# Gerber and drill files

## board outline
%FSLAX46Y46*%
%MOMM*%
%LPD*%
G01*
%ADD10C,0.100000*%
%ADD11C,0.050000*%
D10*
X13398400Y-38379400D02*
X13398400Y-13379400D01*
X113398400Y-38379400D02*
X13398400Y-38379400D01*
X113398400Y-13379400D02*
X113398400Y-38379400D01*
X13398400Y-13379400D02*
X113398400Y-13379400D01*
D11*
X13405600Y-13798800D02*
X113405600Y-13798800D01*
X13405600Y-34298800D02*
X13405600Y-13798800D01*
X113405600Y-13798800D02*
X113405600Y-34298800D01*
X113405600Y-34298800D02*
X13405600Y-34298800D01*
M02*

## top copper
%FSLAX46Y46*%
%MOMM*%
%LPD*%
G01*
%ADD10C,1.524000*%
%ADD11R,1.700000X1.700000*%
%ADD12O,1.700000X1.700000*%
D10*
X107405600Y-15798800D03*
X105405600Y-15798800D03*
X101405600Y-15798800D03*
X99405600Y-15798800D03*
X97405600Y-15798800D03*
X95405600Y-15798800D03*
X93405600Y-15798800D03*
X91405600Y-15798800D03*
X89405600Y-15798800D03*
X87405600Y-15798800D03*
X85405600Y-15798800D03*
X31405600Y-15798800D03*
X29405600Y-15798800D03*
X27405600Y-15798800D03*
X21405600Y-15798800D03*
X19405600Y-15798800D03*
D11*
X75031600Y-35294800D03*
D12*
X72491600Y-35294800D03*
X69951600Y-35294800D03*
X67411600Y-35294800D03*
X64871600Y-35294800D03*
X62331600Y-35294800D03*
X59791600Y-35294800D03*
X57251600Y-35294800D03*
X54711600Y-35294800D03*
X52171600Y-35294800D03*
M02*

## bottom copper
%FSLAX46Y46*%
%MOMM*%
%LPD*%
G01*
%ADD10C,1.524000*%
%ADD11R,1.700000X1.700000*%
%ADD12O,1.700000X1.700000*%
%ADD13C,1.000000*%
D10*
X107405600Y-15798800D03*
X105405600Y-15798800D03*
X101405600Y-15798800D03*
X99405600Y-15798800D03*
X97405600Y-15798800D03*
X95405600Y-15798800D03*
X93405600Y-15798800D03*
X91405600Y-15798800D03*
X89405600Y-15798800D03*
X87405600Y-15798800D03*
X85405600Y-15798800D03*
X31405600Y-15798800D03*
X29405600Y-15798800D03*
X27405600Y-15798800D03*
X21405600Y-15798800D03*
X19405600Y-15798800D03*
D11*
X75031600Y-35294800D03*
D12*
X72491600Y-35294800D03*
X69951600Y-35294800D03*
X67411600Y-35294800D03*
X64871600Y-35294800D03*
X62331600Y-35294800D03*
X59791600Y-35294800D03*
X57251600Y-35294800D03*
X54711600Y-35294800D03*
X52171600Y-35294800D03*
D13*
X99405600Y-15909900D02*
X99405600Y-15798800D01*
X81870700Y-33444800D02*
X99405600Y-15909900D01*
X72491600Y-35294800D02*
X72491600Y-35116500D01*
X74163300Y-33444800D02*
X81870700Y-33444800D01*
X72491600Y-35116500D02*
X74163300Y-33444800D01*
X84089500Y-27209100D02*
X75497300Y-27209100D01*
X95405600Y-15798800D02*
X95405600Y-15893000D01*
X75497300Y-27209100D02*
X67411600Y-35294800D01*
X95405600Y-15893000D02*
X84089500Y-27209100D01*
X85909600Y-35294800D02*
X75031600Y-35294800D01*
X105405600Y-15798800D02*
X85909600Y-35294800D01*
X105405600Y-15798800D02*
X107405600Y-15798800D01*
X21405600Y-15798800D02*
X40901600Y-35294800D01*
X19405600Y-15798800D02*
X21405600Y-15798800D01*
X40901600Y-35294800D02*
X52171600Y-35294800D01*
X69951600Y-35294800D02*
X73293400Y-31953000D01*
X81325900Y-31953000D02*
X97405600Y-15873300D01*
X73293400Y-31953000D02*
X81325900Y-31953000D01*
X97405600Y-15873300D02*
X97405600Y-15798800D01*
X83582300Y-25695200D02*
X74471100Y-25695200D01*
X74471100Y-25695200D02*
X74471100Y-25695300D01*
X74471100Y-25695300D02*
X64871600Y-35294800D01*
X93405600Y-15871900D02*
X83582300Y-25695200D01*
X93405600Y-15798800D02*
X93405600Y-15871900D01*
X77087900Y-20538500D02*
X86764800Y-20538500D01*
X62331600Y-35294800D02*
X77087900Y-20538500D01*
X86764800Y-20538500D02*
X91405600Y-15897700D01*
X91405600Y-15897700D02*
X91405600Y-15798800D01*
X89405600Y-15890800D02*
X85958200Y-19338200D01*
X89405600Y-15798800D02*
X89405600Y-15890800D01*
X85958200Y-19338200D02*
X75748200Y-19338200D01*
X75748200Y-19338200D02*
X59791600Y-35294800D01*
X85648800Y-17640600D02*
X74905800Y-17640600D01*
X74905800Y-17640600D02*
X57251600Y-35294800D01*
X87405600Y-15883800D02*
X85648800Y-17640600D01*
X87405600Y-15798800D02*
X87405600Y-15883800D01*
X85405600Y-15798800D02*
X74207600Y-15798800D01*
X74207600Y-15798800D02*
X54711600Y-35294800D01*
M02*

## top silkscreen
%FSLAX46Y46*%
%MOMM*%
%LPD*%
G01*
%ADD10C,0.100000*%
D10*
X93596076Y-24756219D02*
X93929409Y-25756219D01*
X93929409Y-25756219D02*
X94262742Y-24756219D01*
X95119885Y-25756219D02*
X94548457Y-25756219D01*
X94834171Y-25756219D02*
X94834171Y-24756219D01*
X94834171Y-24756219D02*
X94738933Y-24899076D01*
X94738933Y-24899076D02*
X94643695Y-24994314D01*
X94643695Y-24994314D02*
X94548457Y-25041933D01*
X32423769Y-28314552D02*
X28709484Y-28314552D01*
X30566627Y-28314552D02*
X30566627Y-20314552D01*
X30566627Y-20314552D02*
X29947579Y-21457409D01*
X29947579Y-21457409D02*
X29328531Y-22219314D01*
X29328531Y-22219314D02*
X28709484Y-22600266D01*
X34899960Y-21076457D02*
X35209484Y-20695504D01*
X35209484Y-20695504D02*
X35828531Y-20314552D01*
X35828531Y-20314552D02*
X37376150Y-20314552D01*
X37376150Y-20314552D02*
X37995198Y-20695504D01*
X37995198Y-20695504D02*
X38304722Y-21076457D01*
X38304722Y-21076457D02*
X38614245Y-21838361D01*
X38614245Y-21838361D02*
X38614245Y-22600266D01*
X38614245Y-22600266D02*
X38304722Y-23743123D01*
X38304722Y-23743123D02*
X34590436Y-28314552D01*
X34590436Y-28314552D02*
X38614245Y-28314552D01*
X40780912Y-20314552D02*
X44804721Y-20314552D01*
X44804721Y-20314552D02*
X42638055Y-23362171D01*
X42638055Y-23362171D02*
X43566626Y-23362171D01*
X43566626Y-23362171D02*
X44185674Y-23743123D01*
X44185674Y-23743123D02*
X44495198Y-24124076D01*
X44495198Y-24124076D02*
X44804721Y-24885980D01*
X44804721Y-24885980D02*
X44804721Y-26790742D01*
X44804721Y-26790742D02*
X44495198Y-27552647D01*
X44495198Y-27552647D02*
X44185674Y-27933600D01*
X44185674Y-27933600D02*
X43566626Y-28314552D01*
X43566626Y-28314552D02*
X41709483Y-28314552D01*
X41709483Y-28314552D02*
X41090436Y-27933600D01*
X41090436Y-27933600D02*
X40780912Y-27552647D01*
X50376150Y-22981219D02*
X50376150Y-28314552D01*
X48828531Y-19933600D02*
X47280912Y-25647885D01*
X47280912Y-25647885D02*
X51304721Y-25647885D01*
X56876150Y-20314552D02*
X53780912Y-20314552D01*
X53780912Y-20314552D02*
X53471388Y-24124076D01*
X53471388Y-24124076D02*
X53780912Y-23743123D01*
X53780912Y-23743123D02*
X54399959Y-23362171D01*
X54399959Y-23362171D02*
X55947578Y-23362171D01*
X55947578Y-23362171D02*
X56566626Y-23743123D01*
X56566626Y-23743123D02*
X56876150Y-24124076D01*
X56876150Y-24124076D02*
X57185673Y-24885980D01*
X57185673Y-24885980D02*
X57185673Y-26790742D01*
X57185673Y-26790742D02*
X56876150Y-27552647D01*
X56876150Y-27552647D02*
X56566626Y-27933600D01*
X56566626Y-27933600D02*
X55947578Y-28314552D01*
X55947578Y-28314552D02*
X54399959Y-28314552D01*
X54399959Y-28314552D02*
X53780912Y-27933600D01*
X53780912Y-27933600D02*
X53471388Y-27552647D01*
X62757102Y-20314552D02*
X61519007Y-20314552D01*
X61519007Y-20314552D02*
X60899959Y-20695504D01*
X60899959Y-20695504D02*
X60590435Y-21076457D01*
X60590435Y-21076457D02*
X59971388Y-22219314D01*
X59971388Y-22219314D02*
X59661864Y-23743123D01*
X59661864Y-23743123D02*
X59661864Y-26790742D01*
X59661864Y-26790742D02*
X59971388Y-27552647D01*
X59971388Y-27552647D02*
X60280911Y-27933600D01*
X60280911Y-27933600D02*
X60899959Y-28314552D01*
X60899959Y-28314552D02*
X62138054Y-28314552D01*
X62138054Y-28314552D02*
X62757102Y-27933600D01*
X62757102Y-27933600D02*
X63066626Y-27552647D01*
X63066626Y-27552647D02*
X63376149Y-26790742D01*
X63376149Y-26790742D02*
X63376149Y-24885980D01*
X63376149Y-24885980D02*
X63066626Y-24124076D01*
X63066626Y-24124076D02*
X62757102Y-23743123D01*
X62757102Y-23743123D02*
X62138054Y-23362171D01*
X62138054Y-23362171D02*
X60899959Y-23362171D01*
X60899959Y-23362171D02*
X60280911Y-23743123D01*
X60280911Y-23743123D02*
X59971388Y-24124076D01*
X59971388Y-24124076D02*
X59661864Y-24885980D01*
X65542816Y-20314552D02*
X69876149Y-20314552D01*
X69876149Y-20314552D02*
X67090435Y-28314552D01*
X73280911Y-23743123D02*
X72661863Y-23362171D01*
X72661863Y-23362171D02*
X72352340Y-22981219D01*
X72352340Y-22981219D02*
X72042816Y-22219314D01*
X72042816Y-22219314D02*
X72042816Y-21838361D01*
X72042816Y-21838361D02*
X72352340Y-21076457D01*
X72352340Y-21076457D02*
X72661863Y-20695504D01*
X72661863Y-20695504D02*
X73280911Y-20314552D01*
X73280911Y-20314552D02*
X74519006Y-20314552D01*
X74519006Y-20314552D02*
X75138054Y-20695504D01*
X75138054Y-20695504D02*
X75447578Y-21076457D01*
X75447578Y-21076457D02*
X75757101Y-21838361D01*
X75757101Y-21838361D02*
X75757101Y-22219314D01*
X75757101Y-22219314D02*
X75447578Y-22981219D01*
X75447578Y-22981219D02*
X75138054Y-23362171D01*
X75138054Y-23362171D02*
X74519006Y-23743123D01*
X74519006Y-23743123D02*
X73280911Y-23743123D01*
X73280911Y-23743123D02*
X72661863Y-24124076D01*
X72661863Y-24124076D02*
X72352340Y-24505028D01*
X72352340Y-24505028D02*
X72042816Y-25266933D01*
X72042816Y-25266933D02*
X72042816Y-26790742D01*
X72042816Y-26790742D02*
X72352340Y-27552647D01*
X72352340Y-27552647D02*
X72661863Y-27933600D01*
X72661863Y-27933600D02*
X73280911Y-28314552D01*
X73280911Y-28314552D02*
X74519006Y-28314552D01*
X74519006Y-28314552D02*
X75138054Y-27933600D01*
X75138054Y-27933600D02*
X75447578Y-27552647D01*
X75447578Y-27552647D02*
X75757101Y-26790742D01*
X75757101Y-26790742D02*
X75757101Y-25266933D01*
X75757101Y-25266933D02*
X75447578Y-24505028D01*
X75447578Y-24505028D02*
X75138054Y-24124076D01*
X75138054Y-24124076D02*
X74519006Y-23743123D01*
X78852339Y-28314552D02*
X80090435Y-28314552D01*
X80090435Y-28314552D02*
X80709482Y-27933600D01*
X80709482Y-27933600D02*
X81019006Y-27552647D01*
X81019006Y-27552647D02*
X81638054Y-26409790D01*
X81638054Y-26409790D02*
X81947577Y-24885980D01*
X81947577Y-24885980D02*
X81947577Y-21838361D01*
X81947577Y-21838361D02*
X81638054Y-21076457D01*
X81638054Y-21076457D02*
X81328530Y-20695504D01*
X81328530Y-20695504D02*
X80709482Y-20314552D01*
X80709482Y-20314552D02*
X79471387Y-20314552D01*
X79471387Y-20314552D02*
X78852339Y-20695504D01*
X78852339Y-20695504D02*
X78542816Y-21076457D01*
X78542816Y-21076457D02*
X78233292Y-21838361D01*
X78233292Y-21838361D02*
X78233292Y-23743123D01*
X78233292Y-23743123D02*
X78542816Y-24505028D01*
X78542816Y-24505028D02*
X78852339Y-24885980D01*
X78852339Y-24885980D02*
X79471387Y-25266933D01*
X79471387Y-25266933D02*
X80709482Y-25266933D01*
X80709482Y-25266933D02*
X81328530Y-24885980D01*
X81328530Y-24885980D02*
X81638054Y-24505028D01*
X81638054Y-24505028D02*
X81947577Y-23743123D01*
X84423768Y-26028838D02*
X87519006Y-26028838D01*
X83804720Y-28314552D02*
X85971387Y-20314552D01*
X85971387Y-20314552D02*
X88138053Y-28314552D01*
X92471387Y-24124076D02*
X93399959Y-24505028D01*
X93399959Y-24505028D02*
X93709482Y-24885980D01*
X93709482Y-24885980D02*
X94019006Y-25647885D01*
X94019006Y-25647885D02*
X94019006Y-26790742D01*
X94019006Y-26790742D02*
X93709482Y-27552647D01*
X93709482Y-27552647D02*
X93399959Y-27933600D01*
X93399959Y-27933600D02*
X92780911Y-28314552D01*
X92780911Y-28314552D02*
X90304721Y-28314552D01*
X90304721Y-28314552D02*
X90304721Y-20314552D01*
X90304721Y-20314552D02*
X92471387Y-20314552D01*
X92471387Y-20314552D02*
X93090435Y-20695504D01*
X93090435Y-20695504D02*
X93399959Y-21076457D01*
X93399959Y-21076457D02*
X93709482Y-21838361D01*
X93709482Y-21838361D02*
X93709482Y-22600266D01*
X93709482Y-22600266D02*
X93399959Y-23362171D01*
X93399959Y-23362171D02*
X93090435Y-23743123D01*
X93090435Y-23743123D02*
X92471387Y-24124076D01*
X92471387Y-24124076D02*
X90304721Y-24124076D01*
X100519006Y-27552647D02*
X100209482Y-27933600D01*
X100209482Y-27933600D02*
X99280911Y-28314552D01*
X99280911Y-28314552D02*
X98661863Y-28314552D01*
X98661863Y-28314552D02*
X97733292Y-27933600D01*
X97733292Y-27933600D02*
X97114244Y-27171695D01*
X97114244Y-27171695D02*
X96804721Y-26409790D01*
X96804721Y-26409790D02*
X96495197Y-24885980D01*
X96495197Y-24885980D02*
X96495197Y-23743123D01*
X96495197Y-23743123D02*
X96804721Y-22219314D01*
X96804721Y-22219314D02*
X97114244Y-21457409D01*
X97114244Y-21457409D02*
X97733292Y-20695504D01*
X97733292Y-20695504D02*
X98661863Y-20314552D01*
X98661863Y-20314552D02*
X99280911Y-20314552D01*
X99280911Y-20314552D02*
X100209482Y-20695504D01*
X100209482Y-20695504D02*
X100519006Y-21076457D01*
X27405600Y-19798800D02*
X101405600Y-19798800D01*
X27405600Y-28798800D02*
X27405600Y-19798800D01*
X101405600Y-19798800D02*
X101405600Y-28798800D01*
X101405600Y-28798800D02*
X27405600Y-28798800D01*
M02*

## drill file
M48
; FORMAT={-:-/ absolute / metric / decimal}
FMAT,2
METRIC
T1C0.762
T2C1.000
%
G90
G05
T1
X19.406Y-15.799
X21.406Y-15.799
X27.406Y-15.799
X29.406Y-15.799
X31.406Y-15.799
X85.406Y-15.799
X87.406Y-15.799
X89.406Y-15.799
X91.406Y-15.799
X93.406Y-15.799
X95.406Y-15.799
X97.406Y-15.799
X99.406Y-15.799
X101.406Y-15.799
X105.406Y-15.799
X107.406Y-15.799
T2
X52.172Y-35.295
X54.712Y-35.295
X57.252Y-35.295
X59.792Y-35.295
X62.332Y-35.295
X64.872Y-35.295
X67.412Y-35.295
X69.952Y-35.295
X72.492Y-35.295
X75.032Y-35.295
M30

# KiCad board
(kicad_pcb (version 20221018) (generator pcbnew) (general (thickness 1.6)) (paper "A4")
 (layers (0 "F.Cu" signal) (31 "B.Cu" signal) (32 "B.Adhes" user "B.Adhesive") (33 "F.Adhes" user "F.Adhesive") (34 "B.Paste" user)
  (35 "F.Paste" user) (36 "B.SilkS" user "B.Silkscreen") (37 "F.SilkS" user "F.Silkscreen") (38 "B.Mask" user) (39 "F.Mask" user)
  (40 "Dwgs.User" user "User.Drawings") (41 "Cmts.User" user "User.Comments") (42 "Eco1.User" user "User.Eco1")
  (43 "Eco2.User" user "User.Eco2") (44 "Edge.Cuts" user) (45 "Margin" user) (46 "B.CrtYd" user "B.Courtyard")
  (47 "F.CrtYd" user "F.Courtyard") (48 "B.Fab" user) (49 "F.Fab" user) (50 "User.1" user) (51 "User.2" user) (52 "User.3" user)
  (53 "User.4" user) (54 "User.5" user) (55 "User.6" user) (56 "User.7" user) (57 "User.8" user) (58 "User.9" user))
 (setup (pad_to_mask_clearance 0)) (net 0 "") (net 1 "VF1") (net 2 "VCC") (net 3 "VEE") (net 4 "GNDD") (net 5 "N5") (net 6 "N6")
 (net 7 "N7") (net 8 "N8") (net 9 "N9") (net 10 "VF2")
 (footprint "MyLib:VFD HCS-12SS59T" (layer "F.Cu") (at 13.3056 13.9988)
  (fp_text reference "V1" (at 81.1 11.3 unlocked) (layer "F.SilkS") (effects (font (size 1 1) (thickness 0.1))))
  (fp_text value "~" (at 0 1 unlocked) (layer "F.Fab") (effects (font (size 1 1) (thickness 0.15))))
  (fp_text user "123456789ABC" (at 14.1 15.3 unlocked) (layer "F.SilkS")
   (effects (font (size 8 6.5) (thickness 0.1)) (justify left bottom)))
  (fp_line (start 14.1 5.8) (end 88.1 5.8) (stroke (width 0.1) (type default)) (layer "F.SilkS"))
  (fp_line (start 14.1 14.8) (end 14.1 5.8) (stroke (width 0.1) (type default)) (layer "F.SilkS"))
  (fp_line (start 88.1 5.8) (end 88.1 14.8) (stroke (width 0.1) (type default)) (layer "F.SilkS"))
  (fp_line (start 88.1 14.8) (end 14.1 14.8) (stroke (width 0.1) (type default)) (layer "F.SilkS"))
  (fp_line (start 0.1 -0.2) (end 100.1 -0.2) (stroke (width 0.05) (type default)) (layer "Edge.Cuts"))
  (fp_line (start 0.1 20.3) (end 0.1 -0.2) (stroke (width 0.05) (type default)) (layer "Edge.Cuts"))
  (fp_line (start 100.1 -0.2) (end 100.1 20.3) (stroke (width 0.05) (type default)) (layer "Edge.Cuts"))
  (fp_line (start 100.1 20.3) (end 0.1 20.3) (stroke (width 0.05) (type default)) (layer "Edge.Cuts"))
  (pad "1" thru_hole circle (at 94.1 1.8) (size 1.524 1.524) (drill 0.762) (layers "*.Cu" "*.Mask") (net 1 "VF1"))
  (pad "2" thru_hole circle (at 92.1 1.8) (size 1.524 1.524) (drill 0.762) (layers "*.Cu" "*.Mask") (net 1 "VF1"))
  (pad "4" thru_hole circle (at 88.1 1.8) (size 1.524 1.524) (drill 0.762) (layers "*.Cu" "*.Mask"))
  (pad "5" thru_hole circle (at 86.1 1.8) (size 1.524 1.524) (drill 0.762) (layers "*.Cu" "*.Mask") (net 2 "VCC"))
  (pad "6" thru_hole circle (at 84.1 1.8) (size 1.524 1.524) (drill 0.762) (layers "*.Cu" "*.Mask") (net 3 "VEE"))
  (pad "7" thru_hole circle (at 82.1 1.8) (size 1.524 1.524) (drill 0.762) (layers "*.Cu" "*.Mask") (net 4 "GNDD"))
  (pad "8" thru_hole circle (at 80.1 1.8) (size 1.524 1.524) (drill 0.762) (layers "*.Cu" "*.Mask") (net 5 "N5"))
  (pad "9" thru_hole circle (at 78.1 1.8) (size 1.524 1.524) (drill 0.762) (layers "*.Cu" "*.Mask") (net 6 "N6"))
  (pad "10" thru_hole circle (at 76.1 1.8) (size 1.524 1.524) (drill 0.762) (layers "*.Cu" "*.Mask") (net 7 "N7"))
  (pad "11" thru_hole circle (at 74.1 1.8) (size 1.524 1.524) (drill 0.762) (layers "*.Cu" "*.Mask") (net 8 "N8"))
  (pad "12" thru_hole circle (at 72.1 1.8) (size 1.524 1.524) (drill 0.762) (layers "*.Cu" "*.Mask") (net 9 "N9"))
  (pad "39" thru_hole circle (at 18.1 1.8) (size 1.524 1.524) (drill 0.762) (layers "*.Cu" "*.Mask"))
  (pad "40" thru_hole circle (at 16.1 1.8) (size 1.524 1.524) (drill 0.762) (layers "*.Cu" "*.Mask"))
  (pad "41" thru_hole circle (at 14.1 1.8) (size 1.524 1.524) (drill 0.762) (layers "*.Cu" "*.Mask"))
  (pad "44" thru_hole circle (at 8.1 1.8) (size 1.524 1.524) (drill 0.762) (layers "*.Cu" "*.Mask") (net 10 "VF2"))
  (pad "45" thru_hole circle (at 6.1 1.8) (size 1.524 1.524) (drill 0.762) (layers "*.Cu" "*.Mask") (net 10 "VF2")))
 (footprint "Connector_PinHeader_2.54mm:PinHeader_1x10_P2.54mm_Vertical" (layer "B.Cu") (at 75.0316 35.2948 90)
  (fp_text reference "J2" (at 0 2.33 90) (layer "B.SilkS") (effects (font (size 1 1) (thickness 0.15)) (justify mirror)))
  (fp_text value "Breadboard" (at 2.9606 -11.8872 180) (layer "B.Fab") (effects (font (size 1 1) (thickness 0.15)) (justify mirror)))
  (pad "1" thru_hole rect (at 0 0 90) (size 1.7 1.7) (drill 1) (layers "*.Cu" "*.Mask") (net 1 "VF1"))
  (pad "2" thru_hole oval (at 0 -2.54 90) (size 1.7 1.7) (drill 1) (layers "*.Cu" "*.Mask") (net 2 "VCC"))
  (pad "3" thru_hole oval (at 0 -5.08 90) (size 1.7 1.7) (drill 1) (layers "*.Cu" "*.Mask") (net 3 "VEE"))
  (pad "4" thru_hole oval (at 0 -7.62 90) (size 1.7 1.7) (drill 1) (layers "*.Cu" "*.Mask") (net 4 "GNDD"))
  (pad "5" thru_hole oval (at 0 -10.16 90) (size 1.7 1.7) (drill 1) (layers "*.Cu" "*.Mask") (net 5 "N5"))
  (pad "6" thru_hole oval (at 0 -12.7 90) (size 1.7 1.7) (drill 1) (layers "*.Cu" "*.Mask") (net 6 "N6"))
  (pad "7" thru_hole oval (at 0 -15.24 90) (size 1.7 1.7) (drill 1) (layers "*.Cu" "*.Mask") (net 7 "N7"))
  (pad "8" thru_hole oval (at 0 -17.78 90) (size 1.7 1.7) (drill 1) (layers "*.Cu" "*.Mask") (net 8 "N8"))
  (pad "9" thru_hole oval (at 0 -20.32 90) (size 1.7 1.7) (drill 1) (layers "*.Cu" "*.Mask") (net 9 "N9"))
  (pad "10" thru_hole oval (at 0 -22.86 90) (size 1.7 1.7) (drill 1) (layers "*.Cu" "*.Mask") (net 10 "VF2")))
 (gr_line (start 13.3984 38.3794) (end 13.3984 13.3794) (stroke (width 0.1) (type default)) (layer "Edge.Cuts"))
 (gr_line (start 113.3984 38.3794) (end 13.3984 38.3794) (stroke (width 0.1) (type default)) (layer "Edge.Cuts"))
 (gr_line (start 113.3984 13.3794) (end 113.3984 38.3794) (stroke (width 0.1) (type default)) (layer "Edge.Cuts"))
 (gr_line (start 13.3984 13.3794) (end 113.3984 13.3794) (stroke (width 0.1) (type default)) (layer "Edge.Cuts"))
 (segment (start 99.4056 15.9099) (end 99.4056 15.7988) (width 1) (layer "B.Cu") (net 2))
 (segment (start 81.8707 33.4448) (end 99.4056 15.9099) (width 1) (layer "B.Cu") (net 2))
 (segment (start 72.4916 35.2948) (end 72.4916 35.1165) (width 1) (layer "B.Cu") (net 2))
 (segment (start 74.1633 33.4448) (end 81.8707 33.4448) (width 1) (layer "B.Cu") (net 2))
 (segment (start 72.4916 35.1165) (end 74.1633 33.4448) (width 1) (layer "B.Cu") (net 2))
 (segment (start 84.0895 27.2091) (end 75.4973 27.2091) (width 1) (layer "B.Cu") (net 4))
 (segment (start 95.4056 15.7988) (end 95.4056 15.893) (width 1) (layer "B.Cu") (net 4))
 (segment (start 75.4973 27.2091) (end 67.4116 35.2948) (width 1) (layer "B.Cu") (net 4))
 (segment (start 95.4056 15.893) (end 84.0895 27.2091) (width 1) (layer "B.Cu") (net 4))
 (segment (start 85.9096 35.2948) (end 75.0316 35.2948) (width 1) (layer "B.Cu") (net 1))
 (segment (start 105.4056 15.7988) (end 85.9096 35.2948) (width 1) (layer "B.Cu") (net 1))
 (segment (start 105.4056 15.7988) (end 107.4056 15.7988) (width 1) (layer "B.Cu") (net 1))
 (segment (start 21.4056 15.7988) (end 40.9016 35.2948) (width 1) (layer "B.Cu") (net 10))
 (segment (start 19.4056 15.7988) (end 21.4056 15.7988) (width 1) (layer "B.Cu") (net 10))
 (segment (start 40.9016 35.2948) (end 52.1716 35.2948) (width 1) (layer "B.Cu") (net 10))
 (segment (start 69.9516 35.2948) (end 73.2934 31.953) (width 1) (layer "B.Cu") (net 3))
 (segment (start 81.3259 31.953) (end 97.4056 15.8733) (width 1) (layer "B.Cu") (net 3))
 (segment (start 73.2934 31.953) (end 81.3259 31.953) (width 1) (layer "B.Cu") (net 3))
 (segment (start 97.4056 15.8733) (end 97.4056 15.7988) (width 1) (layer "B.Cu") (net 3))
 (segment (start 83.5823 25.6952) (end 74.4711 25.6952) (width 1) (layer "B.Cu") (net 5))
 (segment (start 74.4711 25.6952) (end 74.4711 25.6953) (width 1) (layer "B.Cu") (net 5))
 (segment (start 74.4711 25.6953) (end 64.8716 35.2948) (width 1) (layer "B.Cu") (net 5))
 (segment (start 93.4056 15.8719) (end 83.5823 25.6952) (width 1) (layer "B.Cu") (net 5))
 (segment (start 93.4056 15.7988) (end 93.4056 15.8719) (width 1) (layer "B.Cu") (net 5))
 (segment (start 77.0879 20.5385) (end 86.7648 20.5385) (width 1) (layer "B.Cu") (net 6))
 (segment (start 62.3316 35.2948) (end 77.0879 20.5385) (width 1) (layer "B.Cu") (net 6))
 (segment (start 86.7648 20.5385) (end 91.4056 15.8977) (width 1) (layer "B.Cu") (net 6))
 (segment (start 91.4056 15.8977) (end 91.4056 15.7988) (width 1) (layer "B.Cu") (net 6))
 (segment (start 89.4056 15.8908) (end 85.9582 19.3382) (width 1) (layer "B.Cu") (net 7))
 (segment (start 89.4056 15.7988) (end 89.4056 15.8908) (width 1) (layer "B.Cu") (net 7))
 (segment (start 85.9582 19.3382) (end 75.7482 19.3382) (width 1) (layer "B.Cu") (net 7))
 (segment (start 75.7482 19.3382) (end 59.7916 35.2948) (width 1) (layer "B.Cu") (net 7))
 (segment (start 85.6488 17.6406) (end 74.9058 17.6406) (width 1) (layer "B.Cu") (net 8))
 (segment (start 74.9058 17.6406) (end 57.2516 35.2948) (width 1) (layer "B.Cu") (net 8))
 (segment (start 87.4056 15.8838) (end 85.6488 17.6406) (width 1) (layer "B.Cu") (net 8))
 (segment (start 87.4056 15.7988) (end 87.4056 15.8838) (width 1) (layer "B.Cu") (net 8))
 (segment (start 85.4056 15.7988) (end 74.2076 15.7988) (width 1) (layer "B.Cu") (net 9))
 (segment (start 74.2076 15.7988) (end 54.7116 35.2948) (width 1) (layer "B.Cu") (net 9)))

